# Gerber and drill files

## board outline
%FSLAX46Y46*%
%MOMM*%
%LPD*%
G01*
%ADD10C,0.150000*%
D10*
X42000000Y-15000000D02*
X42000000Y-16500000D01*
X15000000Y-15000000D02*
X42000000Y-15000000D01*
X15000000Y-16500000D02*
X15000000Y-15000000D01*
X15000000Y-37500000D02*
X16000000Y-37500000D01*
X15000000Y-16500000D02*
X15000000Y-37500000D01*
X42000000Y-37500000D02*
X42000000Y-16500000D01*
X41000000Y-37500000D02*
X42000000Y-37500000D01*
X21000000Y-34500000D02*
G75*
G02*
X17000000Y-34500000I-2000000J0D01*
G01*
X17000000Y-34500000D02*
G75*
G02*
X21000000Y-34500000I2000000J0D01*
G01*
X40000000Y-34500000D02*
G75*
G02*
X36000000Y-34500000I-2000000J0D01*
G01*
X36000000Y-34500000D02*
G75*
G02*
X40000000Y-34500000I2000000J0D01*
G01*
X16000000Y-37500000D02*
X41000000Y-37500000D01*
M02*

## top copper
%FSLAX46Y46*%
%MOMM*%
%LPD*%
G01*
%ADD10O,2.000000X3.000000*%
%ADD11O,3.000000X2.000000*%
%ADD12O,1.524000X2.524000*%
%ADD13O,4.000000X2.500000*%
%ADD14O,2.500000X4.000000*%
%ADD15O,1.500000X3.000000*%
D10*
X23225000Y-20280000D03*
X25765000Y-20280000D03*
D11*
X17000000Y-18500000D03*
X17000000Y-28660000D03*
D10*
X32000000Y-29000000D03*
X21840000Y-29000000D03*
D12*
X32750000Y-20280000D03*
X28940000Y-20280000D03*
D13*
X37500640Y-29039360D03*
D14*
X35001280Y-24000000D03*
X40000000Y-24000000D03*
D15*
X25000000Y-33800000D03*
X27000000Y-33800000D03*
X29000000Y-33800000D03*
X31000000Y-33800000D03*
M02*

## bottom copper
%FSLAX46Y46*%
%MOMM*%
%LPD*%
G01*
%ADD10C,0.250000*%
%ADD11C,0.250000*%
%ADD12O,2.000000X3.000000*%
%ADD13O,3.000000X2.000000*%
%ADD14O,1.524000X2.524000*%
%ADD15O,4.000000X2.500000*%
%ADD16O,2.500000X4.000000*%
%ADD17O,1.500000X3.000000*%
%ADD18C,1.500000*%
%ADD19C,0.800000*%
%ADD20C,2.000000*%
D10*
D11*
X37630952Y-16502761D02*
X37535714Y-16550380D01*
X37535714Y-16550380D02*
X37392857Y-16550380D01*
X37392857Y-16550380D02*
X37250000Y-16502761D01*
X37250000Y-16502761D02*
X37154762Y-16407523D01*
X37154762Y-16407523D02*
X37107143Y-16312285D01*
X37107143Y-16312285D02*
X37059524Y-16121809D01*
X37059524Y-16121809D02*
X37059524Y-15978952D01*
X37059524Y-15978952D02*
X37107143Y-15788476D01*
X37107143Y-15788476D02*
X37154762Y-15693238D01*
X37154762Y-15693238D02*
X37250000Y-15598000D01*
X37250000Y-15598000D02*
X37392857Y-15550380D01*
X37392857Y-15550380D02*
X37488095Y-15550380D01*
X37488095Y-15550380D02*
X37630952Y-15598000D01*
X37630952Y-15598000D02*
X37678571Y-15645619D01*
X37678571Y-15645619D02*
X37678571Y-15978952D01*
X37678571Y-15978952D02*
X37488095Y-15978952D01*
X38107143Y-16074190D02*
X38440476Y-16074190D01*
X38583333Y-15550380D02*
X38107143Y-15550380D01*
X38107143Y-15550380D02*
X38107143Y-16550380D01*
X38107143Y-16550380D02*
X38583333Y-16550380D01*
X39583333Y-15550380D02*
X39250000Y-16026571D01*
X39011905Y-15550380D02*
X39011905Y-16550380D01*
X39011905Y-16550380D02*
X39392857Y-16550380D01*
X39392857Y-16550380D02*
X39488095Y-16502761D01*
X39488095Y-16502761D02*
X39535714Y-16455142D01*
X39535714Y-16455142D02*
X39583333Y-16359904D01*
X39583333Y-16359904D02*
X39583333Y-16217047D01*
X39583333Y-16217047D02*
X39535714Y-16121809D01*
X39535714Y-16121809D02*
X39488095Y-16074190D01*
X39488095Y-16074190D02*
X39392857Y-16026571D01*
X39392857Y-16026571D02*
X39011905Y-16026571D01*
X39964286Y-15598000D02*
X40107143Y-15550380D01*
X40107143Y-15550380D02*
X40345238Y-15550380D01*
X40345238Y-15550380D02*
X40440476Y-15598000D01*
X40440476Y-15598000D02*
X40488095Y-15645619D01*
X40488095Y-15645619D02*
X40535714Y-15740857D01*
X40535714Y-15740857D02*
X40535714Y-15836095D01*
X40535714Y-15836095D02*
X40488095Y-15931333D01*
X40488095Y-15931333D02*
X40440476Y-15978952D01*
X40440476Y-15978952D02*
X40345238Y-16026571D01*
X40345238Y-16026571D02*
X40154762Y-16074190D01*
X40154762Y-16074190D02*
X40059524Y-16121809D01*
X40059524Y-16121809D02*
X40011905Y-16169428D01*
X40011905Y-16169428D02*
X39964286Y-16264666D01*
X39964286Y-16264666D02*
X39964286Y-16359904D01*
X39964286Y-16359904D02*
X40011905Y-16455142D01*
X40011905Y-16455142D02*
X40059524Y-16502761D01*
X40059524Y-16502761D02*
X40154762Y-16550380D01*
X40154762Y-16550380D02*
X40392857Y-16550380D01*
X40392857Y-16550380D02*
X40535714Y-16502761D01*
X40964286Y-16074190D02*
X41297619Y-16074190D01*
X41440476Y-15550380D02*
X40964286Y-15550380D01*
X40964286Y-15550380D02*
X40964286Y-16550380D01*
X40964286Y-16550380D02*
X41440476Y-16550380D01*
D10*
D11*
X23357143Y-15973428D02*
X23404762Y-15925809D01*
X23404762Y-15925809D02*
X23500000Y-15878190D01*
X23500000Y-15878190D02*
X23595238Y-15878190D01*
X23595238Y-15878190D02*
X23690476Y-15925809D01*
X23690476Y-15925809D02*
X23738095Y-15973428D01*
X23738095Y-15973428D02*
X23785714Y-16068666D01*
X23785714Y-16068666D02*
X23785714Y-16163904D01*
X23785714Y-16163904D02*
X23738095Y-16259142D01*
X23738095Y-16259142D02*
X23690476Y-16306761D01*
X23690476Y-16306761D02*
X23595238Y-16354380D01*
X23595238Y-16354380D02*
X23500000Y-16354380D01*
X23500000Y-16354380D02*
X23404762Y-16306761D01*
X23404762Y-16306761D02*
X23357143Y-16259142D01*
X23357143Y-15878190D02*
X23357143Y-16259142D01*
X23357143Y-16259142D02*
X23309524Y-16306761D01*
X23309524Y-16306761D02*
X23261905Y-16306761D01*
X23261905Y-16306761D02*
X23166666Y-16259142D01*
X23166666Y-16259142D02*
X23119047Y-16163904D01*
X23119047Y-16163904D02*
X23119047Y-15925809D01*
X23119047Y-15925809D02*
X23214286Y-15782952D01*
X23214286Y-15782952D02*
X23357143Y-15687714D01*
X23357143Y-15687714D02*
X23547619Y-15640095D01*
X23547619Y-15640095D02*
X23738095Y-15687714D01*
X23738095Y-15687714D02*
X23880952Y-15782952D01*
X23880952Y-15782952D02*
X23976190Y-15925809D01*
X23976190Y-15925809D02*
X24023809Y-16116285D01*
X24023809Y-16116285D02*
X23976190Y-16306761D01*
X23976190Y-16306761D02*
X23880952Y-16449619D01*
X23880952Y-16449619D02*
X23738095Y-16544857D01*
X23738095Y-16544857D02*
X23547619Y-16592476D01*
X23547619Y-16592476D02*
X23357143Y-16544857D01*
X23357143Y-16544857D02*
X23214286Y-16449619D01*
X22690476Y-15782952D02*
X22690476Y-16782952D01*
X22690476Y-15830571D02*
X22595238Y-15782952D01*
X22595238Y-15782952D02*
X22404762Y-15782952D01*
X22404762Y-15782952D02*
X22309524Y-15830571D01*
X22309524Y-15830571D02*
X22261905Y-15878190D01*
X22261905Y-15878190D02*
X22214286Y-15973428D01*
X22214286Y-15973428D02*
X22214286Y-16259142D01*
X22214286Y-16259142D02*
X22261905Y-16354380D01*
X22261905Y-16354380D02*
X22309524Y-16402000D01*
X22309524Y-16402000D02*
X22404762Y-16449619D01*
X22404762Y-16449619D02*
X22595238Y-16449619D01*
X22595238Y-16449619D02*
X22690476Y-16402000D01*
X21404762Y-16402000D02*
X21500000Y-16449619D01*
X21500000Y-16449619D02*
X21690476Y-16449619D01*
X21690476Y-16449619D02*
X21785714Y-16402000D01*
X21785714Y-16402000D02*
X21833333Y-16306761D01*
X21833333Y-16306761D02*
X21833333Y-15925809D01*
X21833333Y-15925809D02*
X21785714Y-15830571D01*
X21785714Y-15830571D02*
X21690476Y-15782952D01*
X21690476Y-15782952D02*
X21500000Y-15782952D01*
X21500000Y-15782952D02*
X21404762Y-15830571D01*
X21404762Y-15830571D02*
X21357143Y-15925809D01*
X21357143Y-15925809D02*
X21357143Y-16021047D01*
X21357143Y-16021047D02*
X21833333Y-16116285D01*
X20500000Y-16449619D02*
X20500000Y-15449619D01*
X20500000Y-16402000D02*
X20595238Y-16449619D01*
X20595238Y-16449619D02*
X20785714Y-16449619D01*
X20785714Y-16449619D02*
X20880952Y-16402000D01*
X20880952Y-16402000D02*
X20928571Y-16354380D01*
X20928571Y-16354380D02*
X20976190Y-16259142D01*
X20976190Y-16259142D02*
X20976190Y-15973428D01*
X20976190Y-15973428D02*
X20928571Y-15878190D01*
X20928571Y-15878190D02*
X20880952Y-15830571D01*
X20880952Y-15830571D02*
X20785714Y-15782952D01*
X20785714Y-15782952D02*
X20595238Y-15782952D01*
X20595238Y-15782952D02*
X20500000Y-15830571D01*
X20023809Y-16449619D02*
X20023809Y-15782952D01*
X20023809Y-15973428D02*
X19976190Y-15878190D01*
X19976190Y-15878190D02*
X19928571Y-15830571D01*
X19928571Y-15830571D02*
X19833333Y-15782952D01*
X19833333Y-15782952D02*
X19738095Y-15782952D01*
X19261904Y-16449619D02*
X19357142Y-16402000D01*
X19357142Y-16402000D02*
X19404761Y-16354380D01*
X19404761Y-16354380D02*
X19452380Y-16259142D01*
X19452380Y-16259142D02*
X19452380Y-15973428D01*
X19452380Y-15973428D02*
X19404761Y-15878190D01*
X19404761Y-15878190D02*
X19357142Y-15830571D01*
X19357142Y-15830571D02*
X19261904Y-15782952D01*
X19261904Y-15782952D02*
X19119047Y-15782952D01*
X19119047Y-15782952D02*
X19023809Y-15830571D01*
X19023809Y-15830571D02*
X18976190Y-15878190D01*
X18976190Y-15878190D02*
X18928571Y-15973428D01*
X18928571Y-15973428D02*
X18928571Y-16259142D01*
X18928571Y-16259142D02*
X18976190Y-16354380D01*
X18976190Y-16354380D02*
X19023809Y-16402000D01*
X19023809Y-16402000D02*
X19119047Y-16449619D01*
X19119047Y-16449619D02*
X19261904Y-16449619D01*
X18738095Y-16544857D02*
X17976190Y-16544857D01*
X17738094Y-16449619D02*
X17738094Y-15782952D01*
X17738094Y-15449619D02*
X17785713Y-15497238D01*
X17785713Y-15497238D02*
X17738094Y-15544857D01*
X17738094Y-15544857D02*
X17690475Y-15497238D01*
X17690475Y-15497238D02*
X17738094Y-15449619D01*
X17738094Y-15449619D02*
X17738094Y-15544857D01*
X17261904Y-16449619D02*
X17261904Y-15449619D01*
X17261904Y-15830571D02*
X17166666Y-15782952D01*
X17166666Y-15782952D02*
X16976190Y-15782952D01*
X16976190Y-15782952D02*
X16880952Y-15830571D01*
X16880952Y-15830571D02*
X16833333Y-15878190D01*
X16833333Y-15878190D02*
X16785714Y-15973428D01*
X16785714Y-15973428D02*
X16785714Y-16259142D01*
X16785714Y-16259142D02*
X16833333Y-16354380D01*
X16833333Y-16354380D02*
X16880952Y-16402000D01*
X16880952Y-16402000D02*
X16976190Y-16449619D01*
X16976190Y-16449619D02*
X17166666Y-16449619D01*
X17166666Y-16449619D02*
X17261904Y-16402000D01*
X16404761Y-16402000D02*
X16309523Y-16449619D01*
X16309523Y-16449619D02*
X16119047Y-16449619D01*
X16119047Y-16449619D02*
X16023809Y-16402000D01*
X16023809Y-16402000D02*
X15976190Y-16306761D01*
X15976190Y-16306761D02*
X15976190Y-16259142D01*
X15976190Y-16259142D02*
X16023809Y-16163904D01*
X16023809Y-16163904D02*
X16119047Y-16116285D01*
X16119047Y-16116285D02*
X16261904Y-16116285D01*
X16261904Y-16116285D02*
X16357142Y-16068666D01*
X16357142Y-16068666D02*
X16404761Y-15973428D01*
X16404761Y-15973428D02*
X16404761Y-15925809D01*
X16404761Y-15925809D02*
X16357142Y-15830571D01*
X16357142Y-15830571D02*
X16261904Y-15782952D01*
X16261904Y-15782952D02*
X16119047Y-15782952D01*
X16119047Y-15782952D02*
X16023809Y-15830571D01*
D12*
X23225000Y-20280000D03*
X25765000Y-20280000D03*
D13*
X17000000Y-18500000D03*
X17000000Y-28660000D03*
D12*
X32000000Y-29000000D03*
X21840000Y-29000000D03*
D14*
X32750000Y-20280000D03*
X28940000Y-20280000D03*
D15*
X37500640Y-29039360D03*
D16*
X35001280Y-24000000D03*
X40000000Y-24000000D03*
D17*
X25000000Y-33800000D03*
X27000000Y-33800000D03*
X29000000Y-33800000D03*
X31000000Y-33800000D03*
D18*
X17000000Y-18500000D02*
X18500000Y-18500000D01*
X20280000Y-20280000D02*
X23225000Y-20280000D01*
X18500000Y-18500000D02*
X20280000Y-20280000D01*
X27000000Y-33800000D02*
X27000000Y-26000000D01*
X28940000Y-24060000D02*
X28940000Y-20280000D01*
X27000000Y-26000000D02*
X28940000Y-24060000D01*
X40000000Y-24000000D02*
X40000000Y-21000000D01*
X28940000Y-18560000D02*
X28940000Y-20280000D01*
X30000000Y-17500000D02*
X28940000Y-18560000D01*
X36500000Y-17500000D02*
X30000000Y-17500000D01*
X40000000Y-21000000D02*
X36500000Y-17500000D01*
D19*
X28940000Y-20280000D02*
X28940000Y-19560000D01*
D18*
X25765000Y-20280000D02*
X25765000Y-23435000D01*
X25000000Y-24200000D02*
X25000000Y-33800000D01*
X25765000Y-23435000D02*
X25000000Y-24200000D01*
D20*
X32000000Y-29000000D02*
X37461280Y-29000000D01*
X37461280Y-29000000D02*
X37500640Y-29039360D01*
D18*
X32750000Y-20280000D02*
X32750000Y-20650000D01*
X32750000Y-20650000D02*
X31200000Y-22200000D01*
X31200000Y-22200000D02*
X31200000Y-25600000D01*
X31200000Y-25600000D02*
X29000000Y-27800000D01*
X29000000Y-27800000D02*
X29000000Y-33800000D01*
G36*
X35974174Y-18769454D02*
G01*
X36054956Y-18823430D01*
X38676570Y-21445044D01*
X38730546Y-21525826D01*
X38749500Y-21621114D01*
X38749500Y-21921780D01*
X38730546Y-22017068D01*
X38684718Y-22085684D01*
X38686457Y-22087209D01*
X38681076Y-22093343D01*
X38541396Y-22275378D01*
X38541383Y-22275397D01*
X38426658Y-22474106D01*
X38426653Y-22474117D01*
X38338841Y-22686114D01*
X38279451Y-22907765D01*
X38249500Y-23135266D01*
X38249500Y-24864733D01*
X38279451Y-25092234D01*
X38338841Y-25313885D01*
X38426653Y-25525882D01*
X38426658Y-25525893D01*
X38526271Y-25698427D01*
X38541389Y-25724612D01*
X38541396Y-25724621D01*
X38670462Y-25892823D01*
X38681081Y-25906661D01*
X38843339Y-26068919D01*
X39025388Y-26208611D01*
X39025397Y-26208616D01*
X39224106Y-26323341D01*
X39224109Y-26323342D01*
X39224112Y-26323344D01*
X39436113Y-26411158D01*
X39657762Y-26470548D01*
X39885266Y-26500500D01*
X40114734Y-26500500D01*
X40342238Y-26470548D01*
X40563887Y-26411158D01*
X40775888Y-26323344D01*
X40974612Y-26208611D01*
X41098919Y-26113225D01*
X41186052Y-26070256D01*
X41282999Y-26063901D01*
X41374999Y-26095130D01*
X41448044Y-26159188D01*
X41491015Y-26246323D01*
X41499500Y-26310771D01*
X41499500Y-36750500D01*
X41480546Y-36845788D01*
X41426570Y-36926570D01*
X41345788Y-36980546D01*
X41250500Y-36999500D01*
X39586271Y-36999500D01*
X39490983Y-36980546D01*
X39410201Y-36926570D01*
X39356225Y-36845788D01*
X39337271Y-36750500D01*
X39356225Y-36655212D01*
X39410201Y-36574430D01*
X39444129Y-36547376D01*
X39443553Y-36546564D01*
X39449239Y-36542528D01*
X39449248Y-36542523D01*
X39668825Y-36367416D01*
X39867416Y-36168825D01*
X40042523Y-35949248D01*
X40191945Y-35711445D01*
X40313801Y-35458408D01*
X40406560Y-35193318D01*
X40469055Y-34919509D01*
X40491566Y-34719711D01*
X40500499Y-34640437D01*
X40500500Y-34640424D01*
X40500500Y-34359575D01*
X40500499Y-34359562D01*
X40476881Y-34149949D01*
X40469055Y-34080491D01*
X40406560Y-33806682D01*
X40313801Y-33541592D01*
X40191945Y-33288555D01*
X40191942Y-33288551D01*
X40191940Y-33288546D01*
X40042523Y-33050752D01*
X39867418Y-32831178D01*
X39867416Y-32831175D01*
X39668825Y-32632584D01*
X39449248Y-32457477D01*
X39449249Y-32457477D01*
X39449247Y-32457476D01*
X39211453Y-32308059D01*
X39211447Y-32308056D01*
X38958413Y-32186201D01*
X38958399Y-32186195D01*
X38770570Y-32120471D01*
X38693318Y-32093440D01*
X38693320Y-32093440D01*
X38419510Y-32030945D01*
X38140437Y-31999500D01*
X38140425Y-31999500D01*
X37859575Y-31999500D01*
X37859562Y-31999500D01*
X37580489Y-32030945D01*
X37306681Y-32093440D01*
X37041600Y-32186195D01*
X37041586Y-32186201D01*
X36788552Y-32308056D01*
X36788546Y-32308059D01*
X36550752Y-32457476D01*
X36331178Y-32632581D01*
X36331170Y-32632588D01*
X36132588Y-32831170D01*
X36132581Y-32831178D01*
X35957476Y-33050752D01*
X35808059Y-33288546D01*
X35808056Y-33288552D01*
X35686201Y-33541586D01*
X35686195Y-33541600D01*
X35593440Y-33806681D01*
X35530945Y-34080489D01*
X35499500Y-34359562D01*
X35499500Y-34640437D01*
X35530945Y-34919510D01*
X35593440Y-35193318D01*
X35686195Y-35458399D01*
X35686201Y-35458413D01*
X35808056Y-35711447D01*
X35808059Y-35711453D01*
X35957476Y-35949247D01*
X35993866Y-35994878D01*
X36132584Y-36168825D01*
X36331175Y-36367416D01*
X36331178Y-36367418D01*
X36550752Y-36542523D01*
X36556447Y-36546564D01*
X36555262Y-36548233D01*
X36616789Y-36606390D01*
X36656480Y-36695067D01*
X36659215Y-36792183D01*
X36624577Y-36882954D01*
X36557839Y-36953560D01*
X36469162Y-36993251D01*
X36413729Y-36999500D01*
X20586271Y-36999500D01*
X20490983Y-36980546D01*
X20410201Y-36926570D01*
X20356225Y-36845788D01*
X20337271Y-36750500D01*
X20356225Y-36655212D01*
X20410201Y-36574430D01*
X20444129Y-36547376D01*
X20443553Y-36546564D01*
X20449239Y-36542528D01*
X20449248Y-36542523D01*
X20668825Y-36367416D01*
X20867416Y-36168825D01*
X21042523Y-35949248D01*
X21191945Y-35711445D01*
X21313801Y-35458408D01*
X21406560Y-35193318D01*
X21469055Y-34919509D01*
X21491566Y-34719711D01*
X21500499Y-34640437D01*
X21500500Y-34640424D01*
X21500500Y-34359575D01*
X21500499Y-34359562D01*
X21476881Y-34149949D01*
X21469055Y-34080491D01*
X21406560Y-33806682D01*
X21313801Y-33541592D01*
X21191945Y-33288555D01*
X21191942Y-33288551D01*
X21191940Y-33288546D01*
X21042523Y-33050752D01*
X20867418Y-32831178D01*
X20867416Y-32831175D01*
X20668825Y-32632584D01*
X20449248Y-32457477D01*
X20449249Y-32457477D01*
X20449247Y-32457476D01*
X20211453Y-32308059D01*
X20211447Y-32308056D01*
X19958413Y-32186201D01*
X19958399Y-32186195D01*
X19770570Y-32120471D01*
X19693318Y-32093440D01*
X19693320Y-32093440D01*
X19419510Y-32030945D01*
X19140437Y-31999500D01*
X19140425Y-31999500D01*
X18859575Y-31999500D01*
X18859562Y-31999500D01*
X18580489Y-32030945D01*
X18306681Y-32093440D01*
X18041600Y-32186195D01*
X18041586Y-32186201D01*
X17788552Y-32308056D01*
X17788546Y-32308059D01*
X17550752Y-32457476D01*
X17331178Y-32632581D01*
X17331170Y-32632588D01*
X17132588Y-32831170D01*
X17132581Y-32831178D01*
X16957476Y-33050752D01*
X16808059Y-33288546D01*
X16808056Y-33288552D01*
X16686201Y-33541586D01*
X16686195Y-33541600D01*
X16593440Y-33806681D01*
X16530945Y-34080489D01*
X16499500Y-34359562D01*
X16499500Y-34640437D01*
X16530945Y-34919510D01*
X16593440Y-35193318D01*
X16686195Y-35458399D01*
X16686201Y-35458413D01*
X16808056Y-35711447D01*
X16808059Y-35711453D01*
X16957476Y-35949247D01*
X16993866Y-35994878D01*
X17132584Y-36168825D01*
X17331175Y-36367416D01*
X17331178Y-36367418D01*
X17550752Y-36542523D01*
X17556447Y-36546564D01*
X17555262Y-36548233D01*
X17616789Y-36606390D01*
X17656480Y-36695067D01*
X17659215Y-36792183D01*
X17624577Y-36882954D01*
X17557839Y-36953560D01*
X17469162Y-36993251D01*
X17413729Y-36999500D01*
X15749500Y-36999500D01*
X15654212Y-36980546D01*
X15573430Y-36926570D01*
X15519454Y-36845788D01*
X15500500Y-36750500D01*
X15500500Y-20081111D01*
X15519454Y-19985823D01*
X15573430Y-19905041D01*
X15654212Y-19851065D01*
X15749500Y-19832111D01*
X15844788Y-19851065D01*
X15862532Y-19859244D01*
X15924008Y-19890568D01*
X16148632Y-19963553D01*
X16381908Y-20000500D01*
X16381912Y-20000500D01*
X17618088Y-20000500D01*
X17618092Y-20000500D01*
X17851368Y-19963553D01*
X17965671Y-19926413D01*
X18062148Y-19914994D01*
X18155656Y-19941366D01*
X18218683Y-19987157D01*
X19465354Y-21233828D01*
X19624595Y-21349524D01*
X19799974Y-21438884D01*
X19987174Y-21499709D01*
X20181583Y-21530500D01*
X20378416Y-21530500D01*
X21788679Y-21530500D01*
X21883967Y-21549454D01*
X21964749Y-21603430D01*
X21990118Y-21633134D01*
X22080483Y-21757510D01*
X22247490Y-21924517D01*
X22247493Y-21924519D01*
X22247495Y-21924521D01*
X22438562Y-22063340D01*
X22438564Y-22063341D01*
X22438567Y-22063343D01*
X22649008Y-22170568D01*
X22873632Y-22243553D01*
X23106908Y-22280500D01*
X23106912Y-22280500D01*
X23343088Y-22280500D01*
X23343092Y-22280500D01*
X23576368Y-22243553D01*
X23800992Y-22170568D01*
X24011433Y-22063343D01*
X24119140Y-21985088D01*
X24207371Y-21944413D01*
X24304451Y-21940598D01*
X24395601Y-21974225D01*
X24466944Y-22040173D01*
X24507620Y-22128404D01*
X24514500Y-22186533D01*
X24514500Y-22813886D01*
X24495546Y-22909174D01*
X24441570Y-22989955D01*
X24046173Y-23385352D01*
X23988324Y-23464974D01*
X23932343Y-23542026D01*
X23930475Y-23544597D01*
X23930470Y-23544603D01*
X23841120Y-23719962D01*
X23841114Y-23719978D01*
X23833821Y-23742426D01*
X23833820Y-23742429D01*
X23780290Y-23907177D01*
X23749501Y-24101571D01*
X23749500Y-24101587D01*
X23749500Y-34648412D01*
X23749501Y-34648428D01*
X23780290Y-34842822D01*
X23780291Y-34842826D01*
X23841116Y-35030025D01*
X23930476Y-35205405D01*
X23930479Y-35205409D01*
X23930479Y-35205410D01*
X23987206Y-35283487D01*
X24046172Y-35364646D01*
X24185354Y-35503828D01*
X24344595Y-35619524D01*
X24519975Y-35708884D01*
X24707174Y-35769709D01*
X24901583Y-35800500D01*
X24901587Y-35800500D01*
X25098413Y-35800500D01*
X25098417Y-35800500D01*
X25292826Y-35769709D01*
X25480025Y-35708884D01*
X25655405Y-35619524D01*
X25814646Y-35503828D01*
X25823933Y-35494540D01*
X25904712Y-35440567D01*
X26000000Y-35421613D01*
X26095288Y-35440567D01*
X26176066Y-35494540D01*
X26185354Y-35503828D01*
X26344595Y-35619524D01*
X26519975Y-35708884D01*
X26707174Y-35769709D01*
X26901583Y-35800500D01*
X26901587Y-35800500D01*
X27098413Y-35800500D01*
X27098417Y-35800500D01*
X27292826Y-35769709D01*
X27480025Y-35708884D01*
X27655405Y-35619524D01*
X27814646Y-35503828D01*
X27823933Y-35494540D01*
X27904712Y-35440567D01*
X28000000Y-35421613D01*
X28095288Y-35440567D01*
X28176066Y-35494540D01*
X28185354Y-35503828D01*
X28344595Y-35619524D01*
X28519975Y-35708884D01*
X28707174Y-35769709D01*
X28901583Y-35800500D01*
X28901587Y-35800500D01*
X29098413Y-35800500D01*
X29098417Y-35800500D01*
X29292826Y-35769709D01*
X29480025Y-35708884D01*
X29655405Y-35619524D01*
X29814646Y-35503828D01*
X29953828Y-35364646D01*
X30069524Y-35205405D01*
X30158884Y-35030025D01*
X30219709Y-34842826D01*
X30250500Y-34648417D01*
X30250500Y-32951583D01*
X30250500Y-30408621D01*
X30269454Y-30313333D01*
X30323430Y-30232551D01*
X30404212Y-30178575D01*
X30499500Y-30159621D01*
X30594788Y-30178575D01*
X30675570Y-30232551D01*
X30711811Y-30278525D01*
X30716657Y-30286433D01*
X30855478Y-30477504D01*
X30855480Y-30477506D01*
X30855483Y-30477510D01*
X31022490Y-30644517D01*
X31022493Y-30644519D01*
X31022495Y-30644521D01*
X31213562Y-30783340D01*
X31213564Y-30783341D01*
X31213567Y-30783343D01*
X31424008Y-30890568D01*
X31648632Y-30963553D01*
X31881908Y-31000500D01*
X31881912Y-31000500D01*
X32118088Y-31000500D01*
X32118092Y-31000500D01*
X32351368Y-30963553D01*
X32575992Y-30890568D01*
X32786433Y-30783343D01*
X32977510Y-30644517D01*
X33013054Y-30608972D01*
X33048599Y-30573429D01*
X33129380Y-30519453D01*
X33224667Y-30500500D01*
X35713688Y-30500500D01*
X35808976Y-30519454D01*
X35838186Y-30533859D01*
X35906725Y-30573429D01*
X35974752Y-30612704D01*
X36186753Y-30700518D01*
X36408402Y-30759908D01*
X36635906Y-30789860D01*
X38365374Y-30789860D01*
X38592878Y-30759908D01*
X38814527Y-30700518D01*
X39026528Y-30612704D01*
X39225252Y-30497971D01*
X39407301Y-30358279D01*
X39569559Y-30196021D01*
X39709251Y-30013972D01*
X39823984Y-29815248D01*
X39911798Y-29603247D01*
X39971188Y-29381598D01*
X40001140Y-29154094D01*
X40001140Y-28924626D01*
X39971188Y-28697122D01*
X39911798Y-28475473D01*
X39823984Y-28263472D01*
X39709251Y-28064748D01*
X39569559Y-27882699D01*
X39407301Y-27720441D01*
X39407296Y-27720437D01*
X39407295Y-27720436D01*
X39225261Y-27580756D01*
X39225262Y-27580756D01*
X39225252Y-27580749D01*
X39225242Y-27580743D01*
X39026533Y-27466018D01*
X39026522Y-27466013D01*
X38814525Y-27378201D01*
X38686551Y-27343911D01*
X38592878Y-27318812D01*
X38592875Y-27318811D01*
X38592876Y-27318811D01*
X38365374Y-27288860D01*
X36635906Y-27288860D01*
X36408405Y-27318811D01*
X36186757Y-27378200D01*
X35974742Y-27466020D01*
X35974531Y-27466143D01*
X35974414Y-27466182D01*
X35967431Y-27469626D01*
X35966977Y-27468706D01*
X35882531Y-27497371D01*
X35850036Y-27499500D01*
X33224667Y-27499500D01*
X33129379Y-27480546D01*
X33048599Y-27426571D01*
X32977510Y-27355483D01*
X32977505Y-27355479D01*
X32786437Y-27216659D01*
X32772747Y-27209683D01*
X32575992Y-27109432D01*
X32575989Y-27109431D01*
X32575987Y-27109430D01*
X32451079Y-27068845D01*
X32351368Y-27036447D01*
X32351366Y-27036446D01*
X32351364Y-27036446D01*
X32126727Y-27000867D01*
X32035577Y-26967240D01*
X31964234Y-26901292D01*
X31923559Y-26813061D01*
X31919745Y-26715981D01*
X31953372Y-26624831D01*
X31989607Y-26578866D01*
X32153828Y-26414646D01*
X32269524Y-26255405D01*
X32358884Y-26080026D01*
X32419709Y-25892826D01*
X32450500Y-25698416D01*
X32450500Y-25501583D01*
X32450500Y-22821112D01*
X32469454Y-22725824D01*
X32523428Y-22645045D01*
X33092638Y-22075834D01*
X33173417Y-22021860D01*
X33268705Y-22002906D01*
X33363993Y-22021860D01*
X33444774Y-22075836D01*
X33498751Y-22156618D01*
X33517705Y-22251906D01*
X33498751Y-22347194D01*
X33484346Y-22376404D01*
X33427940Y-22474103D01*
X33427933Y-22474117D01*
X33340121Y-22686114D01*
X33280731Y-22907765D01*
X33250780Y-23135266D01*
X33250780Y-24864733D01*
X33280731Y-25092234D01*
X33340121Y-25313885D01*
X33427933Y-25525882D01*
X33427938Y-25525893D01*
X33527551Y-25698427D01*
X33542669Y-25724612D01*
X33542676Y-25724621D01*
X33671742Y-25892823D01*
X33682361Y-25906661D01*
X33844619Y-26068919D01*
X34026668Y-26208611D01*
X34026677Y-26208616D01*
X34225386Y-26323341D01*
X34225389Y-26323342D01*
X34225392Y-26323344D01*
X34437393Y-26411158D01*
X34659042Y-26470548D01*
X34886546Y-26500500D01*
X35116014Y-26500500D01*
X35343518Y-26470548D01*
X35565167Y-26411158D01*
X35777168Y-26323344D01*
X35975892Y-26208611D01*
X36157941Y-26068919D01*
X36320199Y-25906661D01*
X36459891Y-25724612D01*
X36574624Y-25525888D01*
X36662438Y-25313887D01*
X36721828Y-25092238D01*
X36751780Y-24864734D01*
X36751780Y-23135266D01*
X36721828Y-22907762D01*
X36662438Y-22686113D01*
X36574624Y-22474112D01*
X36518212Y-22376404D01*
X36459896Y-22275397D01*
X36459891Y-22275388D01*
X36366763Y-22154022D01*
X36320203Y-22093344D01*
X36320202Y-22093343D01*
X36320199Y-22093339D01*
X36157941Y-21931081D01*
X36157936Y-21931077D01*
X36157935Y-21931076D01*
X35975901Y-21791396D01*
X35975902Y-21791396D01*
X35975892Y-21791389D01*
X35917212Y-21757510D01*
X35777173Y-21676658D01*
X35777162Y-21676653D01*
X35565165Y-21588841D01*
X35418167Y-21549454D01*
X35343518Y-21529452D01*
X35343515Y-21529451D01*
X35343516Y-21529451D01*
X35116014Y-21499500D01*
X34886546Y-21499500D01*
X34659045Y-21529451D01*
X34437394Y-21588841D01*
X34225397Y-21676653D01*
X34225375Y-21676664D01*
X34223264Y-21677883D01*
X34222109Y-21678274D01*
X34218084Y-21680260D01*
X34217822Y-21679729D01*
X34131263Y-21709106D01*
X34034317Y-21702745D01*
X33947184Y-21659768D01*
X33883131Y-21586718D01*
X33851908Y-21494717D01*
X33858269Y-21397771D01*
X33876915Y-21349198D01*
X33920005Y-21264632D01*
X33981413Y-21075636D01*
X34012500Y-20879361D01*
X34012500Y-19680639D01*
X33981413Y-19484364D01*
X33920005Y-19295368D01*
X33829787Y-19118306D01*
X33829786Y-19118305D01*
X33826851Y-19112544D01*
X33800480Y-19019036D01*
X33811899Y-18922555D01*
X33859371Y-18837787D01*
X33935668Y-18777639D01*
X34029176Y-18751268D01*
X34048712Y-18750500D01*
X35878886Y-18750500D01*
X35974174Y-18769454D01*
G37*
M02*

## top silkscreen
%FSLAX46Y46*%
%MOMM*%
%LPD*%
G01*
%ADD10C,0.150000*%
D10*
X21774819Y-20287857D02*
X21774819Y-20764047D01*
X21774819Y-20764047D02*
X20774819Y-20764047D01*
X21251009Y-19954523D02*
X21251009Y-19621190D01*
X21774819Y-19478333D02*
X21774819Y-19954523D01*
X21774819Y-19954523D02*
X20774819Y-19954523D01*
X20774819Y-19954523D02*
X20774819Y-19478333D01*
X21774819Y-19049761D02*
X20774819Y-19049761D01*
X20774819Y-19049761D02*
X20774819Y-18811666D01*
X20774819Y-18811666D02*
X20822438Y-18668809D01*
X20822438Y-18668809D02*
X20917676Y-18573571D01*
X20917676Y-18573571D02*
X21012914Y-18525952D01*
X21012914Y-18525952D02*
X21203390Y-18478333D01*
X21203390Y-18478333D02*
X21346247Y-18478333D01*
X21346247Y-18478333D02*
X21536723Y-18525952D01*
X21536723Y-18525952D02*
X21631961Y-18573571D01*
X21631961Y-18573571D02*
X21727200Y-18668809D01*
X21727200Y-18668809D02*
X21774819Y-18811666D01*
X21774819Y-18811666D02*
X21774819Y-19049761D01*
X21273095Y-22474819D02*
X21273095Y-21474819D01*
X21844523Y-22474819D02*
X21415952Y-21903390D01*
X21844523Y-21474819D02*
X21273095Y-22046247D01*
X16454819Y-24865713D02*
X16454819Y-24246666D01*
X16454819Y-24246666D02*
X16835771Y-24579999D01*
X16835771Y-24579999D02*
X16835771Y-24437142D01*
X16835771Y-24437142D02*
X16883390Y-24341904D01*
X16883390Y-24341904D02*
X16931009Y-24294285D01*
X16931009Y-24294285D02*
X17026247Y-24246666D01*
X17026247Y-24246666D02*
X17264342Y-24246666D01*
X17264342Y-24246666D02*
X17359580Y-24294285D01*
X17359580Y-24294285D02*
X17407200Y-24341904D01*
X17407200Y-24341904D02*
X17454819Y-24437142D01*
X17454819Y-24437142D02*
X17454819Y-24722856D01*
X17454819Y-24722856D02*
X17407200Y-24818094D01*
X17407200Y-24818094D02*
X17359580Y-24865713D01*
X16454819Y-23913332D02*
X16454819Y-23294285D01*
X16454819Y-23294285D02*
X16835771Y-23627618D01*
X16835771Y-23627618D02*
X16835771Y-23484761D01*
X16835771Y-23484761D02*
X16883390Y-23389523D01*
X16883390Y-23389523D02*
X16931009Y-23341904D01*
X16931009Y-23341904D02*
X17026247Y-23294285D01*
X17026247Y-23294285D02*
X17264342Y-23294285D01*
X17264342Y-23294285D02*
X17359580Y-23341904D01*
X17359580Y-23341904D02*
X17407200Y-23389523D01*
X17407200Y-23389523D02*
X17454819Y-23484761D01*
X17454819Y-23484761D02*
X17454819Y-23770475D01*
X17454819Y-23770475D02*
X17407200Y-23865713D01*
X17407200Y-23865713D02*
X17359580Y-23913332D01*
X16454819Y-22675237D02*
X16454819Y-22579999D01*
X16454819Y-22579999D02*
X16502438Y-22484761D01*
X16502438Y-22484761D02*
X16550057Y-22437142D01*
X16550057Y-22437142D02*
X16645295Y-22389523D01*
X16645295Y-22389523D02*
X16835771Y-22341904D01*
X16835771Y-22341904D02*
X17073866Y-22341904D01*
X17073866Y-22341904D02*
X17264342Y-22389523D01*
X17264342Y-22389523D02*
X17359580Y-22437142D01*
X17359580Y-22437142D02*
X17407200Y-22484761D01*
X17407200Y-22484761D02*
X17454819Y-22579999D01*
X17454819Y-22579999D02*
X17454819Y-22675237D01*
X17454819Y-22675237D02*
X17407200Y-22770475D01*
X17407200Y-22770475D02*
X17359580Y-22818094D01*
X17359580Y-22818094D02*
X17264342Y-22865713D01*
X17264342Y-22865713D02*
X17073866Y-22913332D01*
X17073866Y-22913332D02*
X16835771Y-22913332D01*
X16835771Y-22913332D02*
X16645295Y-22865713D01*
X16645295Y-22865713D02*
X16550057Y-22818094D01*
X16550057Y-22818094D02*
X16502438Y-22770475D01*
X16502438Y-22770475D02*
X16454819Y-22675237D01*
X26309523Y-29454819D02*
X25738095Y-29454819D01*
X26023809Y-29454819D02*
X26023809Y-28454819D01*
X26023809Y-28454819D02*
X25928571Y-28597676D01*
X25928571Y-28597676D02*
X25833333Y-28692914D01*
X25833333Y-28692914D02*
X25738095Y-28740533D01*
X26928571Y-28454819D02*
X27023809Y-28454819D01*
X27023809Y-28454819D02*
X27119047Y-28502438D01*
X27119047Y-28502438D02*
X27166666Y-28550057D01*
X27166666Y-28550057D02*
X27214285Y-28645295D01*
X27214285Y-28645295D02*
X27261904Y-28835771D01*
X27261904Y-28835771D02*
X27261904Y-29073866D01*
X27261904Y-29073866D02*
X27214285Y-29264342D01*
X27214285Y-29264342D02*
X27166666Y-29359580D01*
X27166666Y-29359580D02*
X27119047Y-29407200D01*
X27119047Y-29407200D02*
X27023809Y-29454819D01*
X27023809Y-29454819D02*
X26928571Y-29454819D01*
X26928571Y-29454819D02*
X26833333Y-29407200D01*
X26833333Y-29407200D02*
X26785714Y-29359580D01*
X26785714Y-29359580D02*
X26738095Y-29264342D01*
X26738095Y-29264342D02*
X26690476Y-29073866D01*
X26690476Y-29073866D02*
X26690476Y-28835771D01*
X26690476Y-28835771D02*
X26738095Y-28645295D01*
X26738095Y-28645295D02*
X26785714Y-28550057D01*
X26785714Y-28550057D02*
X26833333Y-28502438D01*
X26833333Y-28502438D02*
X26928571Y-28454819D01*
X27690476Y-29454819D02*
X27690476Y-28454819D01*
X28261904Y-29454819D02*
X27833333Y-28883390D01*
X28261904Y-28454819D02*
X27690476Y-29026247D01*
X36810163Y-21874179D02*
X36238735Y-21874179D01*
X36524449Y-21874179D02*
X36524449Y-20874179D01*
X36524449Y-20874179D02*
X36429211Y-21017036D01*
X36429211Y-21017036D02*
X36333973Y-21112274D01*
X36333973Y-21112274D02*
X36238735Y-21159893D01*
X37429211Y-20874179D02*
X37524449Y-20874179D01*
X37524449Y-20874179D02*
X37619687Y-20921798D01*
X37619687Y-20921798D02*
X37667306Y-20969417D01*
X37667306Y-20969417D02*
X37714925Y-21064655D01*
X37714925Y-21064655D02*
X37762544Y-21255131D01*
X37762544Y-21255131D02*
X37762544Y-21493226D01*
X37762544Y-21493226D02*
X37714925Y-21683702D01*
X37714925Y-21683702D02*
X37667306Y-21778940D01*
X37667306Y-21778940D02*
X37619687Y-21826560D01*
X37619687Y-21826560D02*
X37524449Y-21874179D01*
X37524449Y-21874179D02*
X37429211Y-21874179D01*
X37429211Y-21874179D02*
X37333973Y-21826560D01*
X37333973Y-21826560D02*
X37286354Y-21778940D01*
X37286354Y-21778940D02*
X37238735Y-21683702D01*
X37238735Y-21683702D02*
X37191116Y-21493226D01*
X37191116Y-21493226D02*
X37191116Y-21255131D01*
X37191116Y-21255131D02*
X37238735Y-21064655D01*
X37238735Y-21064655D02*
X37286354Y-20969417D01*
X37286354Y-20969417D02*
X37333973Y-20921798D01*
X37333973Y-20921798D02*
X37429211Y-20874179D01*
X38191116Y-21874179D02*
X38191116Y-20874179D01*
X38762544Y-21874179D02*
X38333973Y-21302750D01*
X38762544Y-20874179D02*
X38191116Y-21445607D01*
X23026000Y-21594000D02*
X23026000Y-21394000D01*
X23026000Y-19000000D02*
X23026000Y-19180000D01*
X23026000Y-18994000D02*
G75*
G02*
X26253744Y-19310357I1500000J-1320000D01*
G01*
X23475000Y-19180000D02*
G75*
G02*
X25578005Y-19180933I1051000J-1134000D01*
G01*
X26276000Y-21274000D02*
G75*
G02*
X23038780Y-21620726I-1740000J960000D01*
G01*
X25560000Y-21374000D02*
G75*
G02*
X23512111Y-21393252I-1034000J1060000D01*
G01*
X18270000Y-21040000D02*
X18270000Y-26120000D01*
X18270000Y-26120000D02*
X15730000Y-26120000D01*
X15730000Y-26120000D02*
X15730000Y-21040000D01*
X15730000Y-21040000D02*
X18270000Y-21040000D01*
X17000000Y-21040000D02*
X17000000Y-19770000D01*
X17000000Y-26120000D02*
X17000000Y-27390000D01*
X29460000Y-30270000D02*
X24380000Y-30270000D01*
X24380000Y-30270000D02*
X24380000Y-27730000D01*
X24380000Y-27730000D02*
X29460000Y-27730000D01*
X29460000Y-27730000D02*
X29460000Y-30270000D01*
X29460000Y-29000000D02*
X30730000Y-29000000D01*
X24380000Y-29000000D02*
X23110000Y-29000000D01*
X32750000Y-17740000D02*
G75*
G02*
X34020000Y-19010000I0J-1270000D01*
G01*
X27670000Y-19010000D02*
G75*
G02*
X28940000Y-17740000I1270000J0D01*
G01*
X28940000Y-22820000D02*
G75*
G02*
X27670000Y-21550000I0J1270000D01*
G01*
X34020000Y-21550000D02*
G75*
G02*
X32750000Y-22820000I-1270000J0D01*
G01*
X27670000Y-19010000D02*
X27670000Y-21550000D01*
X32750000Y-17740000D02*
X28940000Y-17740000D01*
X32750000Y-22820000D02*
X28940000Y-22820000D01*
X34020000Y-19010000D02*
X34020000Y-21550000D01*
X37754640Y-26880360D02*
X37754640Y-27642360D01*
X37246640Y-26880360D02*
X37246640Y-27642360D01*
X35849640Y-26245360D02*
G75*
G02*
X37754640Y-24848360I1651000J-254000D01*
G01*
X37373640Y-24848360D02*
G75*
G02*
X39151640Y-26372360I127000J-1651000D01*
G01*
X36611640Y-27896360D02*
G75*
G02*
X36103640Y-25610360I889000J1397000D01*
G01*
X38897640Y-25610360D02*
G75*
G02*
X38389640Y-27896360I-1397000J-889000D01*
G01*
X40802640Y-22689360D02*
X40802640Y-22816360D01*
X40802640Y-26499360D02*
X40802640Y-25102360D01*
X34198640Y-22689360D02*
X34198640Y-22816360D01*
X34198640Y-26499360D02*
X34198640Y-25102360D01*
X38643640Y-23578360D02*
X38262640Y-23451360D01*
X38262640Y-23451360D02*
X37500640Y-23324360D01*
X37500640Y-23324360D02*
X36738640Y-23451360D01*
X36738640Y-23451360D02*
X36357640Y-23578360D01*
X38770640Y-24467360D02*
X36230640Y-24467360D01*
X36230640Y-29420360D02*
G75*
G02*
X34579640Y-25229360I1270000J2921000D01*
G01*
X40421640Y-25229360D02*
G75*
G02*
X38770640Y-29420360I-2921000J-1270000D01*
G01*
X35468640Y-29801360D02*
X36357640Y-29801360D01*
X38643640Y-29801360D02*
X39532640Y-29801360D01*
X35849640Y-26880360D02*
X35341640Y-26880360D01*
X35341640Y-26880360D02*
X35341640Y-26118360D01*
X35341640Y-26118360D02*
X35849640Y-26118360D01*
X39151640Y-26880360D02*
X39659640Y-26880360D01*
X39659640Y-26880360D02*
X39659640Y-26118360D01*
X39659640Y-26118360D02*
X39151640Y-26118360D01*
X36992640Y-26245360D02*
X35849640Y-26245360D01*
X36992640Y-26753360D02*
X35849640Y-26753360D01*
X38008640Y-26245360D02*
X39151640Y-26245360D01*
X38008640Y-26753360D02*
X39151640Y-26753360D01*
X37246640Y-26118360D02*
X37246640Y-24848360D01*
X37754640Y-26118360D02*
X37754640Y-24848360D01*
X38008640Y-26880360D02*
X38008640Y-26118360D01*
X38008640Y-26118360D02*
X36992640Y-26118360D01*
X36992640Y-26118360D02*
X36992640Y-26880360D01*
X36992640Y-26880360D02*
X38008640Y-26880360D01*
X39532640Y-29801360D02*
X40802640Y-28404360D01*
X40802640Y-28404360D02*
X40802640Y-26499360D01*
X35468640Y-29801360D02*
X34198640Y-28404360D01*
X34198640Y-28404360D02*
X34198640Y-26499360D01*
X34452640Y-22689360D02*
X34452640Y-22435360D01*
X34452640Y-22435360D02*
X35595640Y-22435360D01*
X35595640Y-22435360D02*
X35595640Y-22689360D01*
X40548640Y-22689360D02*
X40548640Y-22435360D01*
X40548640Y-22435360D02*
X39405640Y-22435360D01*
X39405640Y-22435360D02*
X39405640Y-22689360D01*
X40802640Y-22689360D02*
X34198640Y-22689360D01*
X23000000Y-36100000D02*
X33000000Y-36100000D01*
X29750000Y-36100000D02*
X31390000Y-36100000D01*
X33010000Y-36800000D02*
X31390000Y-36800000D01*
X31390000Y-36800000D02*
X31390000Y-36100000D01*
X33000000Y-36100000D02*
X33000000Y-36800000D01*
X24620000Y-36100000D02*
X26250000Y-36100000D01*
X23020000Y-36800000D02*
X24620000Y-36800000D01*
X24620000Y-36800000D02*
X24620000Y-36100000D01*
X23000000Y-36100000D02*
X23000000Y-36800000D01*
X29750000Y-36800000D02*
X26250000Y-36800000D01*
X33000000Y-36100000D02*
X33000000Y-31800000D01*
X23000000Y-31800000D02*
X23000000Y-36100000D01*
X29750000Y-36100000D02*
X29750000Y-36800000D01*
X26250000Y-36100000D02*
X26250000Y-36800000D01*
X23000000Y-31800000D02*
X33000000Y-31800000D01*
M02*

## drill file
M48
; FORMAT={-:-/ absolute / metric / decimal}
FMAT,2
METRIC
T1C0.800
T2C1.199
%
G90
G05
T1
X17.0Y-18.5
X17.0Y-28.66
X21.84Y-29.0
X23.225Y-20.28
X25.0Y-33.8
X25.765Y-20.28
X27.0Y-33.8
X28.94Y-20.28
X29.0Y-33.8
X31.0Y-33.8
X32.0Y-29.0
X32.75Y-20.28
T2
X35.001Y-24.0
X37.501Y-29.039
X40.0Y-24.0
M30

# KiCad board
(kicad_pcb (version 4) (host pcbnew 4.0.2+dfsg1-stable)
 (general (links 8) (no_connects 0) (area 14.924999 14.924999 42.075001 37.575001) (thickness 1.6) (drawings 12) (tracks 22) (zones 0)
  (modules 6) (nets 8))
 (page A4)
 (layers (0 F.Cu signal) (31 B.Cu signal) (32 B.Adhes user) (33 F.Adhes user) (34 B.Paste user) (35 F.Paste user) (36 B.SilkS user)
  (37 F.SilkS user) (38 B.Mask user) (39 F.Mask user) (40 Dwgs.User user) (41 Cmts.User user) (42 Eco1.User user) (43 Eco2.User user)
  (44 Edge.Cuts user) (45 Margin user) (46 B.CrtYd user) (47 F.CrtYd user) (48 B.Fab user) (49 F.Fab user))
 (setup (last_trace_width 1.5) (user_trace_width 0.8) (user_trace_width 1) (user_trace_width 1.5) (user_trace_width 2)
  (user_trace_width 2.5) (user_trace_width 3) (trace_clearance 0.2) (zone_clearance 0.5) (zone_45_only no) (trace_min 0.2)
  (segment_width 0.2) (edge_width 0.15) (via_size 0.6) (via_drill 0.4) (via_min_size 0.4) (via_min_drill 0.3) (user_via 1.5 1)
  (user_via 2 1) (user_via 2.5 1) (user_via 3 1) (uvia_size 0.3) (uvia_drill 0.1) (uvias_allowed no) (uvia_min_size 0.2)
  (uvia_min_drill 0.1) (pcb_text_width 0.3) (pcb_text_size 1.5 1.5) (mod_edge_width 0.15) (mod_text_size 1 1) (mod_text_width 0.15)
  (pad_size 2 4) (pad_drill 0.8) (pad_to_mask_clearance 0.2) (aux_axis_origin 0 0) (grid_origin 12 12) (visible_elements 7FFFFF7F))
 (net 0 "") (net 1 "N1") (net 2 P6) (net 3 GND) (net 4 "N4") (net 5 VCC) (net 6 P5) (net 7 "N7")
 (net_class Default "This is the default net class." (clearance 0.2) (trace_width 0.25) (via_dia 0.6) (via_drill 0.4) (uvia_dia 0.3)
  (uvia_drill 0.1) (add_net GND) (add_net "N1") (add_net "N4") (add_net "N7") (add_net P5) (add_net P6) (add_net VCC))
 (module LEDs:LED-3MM (layer F.Cu) (at 23.225 20.28)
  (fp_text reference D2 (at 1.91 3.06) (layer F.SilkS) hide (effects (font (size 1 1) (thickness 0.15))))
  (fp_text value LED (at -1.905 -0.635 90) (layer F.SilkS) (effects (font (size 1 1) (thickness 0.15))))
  (fp_line (start -0.199 1.314) (end -0.199 1.114) (layer F.SilkS) (width 0.15))
  (fp_line (start -0.199 -1.28) (end -0.199 -1.1) (layer F.SilkS) (width 0.15))
  (fp_arc (start 1.301 0.034) (end -0.199 -1.286) (angle 108.5) (layer F.SilkS) (width 0.15))
  (fp_arc (start 1.301 0.034) (end 0.25 -1.1) (angle 85.7) (layer F.SilkS) (width 0.15))
  (fp_arc (start 1.311 0.034) (end 3.051 0.994) (angle 110) (layer F.SilkS) (width 0.15))
  (fp_arc (start 1.301 0.034) (end 2.335 1.094) (angle 87.5) (layer F.SilkS) (width 0.15))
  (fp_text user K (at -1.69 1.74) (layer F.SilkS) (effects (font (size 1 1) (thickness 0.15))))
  (pad 1 thru_hole oval (at 0 0 90) (size 3 2) (drill 0.8) (layers *.Cu) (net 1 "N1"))
  (pad 2 thru_hole oval (at 2.54 0) (size 2 3) (drill 0.8) (layers *.Cu) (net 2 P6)))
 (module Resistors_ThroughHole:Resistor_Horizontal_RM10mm (layer F.Cu) (at 17 18.5 270)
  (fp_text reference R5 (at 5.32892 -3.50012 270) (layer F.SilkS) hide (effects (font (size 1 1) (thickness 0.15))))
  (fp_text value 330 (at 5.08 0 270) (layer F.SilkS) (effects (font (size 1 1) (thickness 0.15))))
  (fp_line (start 2.54 -1.27) (end 7.62 -1.27) (layer F.SilkS) (width 0.15))
  (fp_line (start 7.62 -1.27) (end 7.62 1.27) (layer F.SilkS) (width 0.15))
  (fp_line (start 7.62 1.27) (end 2.54 1.27) (layer F.SilkS) (width 0.15))
  (fp_line (start 2.54 1.27) (end 2.54 -1.27) (layer F.SilkS) (width 0.15))
  (fp_line (start 2.54 0) (end 1.27 0) (layer F.SilkS) (width 0.15))
  (fp_line (start 7.62 0) (end 8.89 0) (layer F.SilkS) (width 0.15))
  (pad 1 thru_hole oval (at 0 0 270) (size 2 3) (drill 0.8) (layers *.Cu) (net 1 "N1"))
  (pad 2 thru_hole oval (at 10.16 0 270) (size 2 3) (drill 0.8) (layers *.Cu) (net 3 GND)))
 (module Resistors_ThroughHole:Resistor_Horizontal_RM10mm (layer F.Cu) (at 32 29 180)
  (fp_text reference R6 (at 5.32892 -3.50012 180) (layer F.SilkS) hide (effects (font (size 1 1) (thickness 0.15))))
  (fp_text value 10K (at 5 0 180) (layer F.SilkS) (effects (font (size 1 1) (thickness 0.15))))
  (fp_line (start 2.54 -1.27) (end 7.62 -1.27) (layer F.SilkS) (width 0.15))
  (fp_line (start 7.62 -1.27) (end 7.62 1.27) (layer F.SilkS) (width 0.15))
  (fp_line (start 7.62 1.27) (end 2.54 1.27) (layer F.SilkS) (width 0.15))
  (fp_line (start 2.54 1.27) (end 2.54 -1.27) (layer F.SilkS) (width 0.15))
  (fp_line (start 2.54 0) (end 1.27 0) (layer F.SilkS) (width 0.15))
  (fp_line (start 7.62 0) (end 8.89 0) (layer F.SilkS) (width 0.15))
  (pad 1 thru_hole oval (at 0 0 180) (size 2 3) (drill 0.8) (layers *.Cu) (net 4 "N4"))
  (pad 2 thru_hole oval (at 10.16 0 180) (size 2 3) (drill 0.8) (layers *.Cu) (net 3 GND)))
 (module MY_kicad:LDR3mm (layer F.Cu) (at 32.75 20.28 180)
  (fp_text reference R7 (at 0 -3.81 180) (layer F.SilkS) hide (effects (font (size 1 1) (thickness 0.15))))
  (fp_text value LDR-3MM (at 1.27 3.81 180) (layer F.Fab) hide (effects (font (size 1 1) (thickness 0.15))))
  (fp_arc (start 0 1.27) (end 0 2.54) (angle 90) (layer F.SilkS) (width 0.15))
  (fp_arc (start 3.81 1.27) (end 5.08 1.27) (angle 90) (layer F.SilkS) (width 0.15))
  (fp_arc (start 3.81 -1.27) (end 3.81 -2.54) (angle 90) (layer F.SilkS) (width 0.15))
  (fp_arc (start 0 -1.27) (end -1.27 -1.27) (angle 90) (layer F.SilkS) (width 0.15))
  (fp_line (start 5.08 1.27) (end 5.08 -1.27) (layer F.SilkS) (width 0.15))
  (fp_line (start 0 2.54) (end 3.81 2.54) (layer F.SilkS) (width 0.15))
  (fp_line (start 0 -2.54) (end 3.81 -2.54) (layer F.SilkS) (width 0.15))
  (fp_line (start -1.27 1.27) (end -1.27 -1.27) (layer F.SilkS) (width 0.15))
  (pad 1 thru_hole oval (at 0 0 180) (size 1.524 2.524) (drill 0.8) (layers *.Cu) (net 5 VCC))
  (pad 2 thru_hole oval (at 3.81 0 180) (size 1.524 2.524) (drill 0.8) (layers *.Cu) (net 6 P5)))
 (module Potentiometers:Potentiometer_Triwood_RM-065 (layer F.Cu) (at 40 24 180)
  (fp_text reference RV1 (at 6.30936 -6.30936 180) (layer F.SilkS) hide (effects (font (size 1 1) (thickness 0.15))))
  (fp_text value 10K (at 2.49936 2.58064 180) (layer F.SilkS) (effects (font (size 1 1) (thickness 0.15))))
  (fp_line (start 2.24536 -2.88036) (end 2.24536 -3.64236) (layer F.SilkS) (width 0.15))
  (fp_line (start 2.75336 -2.88036) (end 2.75336 -3.64236) (layer F.SilkS) (width 0.15))
  (fp_arc (start 2.49936 -2.49936) (end 4.15036 -2.24536) (angle 90) (layer F.SilkS) (width 0.15))
  (fp_arc (start 2.49936 -2.49936) (end 2.62636 -0.84836) (angle 90) (layer F.SilkS) (width 0.15))
  (fp_arc (start 2.49936 -2.49936) (end 3.38836 -3.89636) (angle 90) (layer F.SilkS) (width 0.15))
  (fp_arc (start 2.49936 -2.49936) (end 1.10236 -1.61036) (angle 90) (layer F.SilkS) (width 0.15))
  (fp_line (start -0.80264 1.31064) (end -0.80264 1.18364) (layer F.SilkS) (width 0.15))
  (fp_line (start -0.80264 -2.49936) (end -0.80264 -1.10236) (layer F.SilkS) (width 0.15))
  (fp_line (start 5.80136 1.31064) (end 5.80136 1.18364) (layer F.SilkS) (width 0.15))
  (fp_line (start 5.80136 -2.49936) (end 5.80136 -1.10236) (layer F.SilkS) (width 0.15))
  (fp_line (start 1.35636 0.42164) (end 1.73736 0.54864) (layer F.SilkS) (width 0.15))
  (fp_line (start 1.73736 0.54864) (end 2.49936 0.67564) (layer F.SilkS) (width 0.15))
  (fp_line (start 2.49936 0.67564) (end 3.26136 0.54864) (layer F.SilkS) (width 0.15))
  (fp_line (start 3.26136 0.54864) (end 3.64236 0.42164) (layer F.SilkS) (width 0.15))
  (fp_line (start 1.22936 -0.46736) (end 3.76936 -0.46736) (layer F.SilkS) (width 0.15))
  (fp_arc (start 2.49936 -2.49936) (end 3.76936 -5.42036) (angle 90) (layer F.SilkS) (width 0.15))
  (fp_arc (start 2.49936 -2.49936) (end -0.42164 -1.22936) (angle 90) (layer F.SilkS) (width 0.15))
  (fp_line (start 4.53136 -5.80136) (end 3.64236 -5.80136) (layer F.SilkS) (width 0.15))
  (fp_line (start 1.35636 -5.80136) (end 0.46736 -5.80136) (layer F.SilkS) (width 0.15))
  (fp_line (start 4.15036 -2.88036) (end 4.65836 -2.88036) (layer F.SilkS) (width 0.15))
  (fp_line (start 4.65836 -2.88036) (end 4.65836 -2.11836) (layer F.SilkS) (width 0.15))
  (fp_line (start 4.65836 -2.11836) (end 4.15036 -2.11836) (layer F.SilkS) (width 0.15))
  (fp_line (start 0.84836 -2.88036) (end 0.34036 -2.88036) (layer F.SilkS) (width 0.15))
  (fp_line (start 0.34036 -2.88036) (end 0.34036 -2.11836) (layer F.SilkS) (width 0.15))
  (fp_line (start 0.34036 -2.11836) (end 0.84836 -2.11836) (layer F.SilkS) (width 0.15))
  (fp_line (start 3.00736 -2.24536) (end 4.15036 -2.24536) (layer F.SilkS) (width 0.15))
  (fp_line (start 3.00736 -2.75336) (end 4.15036 -2.75336) (layer F.SilkS) (width 0.15))
  (fp_line (start 1.99136 -2.24536) (end 0.84836 -2.24536) (layer F.SilkS) (width 0.15))
  (fp_line (start 1.99136 -2.75336) (end 0.84836 -2.75336) (layer F.SilkS) (width 0.15))
  (fp_line (start 2.75336 -2.11836) (end 2.75336 -0.84836) (layer F.SilkS) (width 0.15))
  (fp_line (start 2.24536 -2.11836) (end 2.24536 -0.84836) (layer F.SilkS) (width 0.15))
  (fp_line (start 1.99136 -2.88036) (end 1.99136 -2.11836) (layer F.SilkS) (width 0.15))
  (fp_line (start 1.99136 -2.11836) (end 3.00736 -2.11836) (layer F.SilkS) (width 0.15))
  (fp_line (start 3.00736 -2.11836) (end 3.00736 -2.88036) (layer F.SilkS) (width 0.15))
  (fp_line (start 3.00736 -2.88036) (end 1.99136 -2.88036) (layer F.SilkS) (width 0.15))
  (fp_line (start 0.46736 -5.80136) (end -0.80264 -4.40436) (layer F.SilkS) (width 0.15))
  (fp_line (start -0.80264 -4.40436) (end -0.80264 -2.49936) (layer F.SilkS) (width 0.15))
  (fp_line (start 4.53136 -5.80136) (end 5.80136 -4.40436) (layer F.SilkS) (width 0.15))
  (fp_line (start 5.80136 -4.40436) (end 5.80136 -2.49936) (layer F.SilkS) (width 0.15))
  (fp_line (start 5.54736 1.31064) (end 5.54736 1.56464) (layer F.SilkS) (width 0.15))
  (fp_line (start 5.54736 1.56464) (end 4.40436 1.56464) (layer F.SilkS) (width 0.15))
  (fp_line (start 4.40436 1.56464) (end 4.40436 1.31064) (layer F.SilkS) (width 0.15))
  (fp_line (start -0.54864 1.31064) (end -0.54864 1.56464) (layer F.SilkS) (width 0.15))
  (fp_line (start -0.54864 1.56464) (end 0.59436 1.56464) (layer F.SilkS) (width 0.15))
  (fp_line (start 0.59436 1.56464) (end 0.59436 1.31064) (layer F.SilkS) (width 0.15))
  (fp_line (start -0.80264 1.31064) (end 5.80136 1.31064) (layer F.SilkS) (width 0.15))
  (pad 2 thru_hole oval (at 2.49936 -5.03936 180) (size 4 2.5) (drill 1.19888) (layers *.Cu) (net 4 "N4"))
  (pad 3 thru_hole oval (at 4.99872 0 180) (size 2.5 4) (drill 1.19888) (layers *.Cu) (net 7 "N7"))
  (pad 1 thru_hole oval (at 0 0 180) (size 2.5 4) (drill 1.19888) (layers *.Cu) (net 6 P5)))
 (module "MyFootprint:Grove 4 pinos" (layer F.Cu) (at 28 33.8)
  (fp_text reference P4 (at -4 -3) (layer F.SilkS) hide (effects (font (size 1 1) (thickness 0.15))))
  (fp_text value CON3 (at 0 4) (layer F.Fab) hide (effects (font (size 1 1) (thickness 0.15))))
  (fp_line (start -5 2.3) (end 5 2.3) (layer F.SilkS) (width 0.15))
  (fp_line (start 1.75 2.3) (end 3.39 2.3) (layer F.SilkS) (width 0.15))
  (fp_line (start 5.01 3) (end 3.39 3) (layer F.SilkS) (width 0.15))
  (fp_line (start 3.39 3) (end 3.39 2.3) (layer F.SilkS) (width 0.15))
  (fp_line (start 5 2.3) (end 5 3) (layer F.SilkS) (width 0.15))
  (fp_line (start -3.38 2.3) (end -1.75 2.3) (layer F.SilkS) (width 0.15))
  (fp_line (start -4.98 3) (end -3.38 3) (layer F.SilkS) (width 0.15))
  (fp_line (start -3.38 3) (end -3.38 2.3) (layer F.SilkS) (width 0.15))
  (fp_line (start -5 2.3) (end -5 3) (layer F.SilkS) (width 0.15))
  (fp_line (start 1.75 3) (end -1.75 3) (layer F.SilkS) (width 0.15))
  (fp_line (start 5 2.3) (end 5 -2) (layer F.SilkS) (width 0.15))
  (fp_line (start -5 -2) (end -5 2.3) (layer F.SilkS) (width 0.15))
  (fp_line (start 1.75 2.3) (end 1.75 3) (layer F.SilkS) (width 0.15))
  (fp_line (start -1.75 2.3) (end -1.75 3) (layer F.SilkS) (width 0.15))
  (fp_line (start -5 -2) (end 5 -2) (layer F.SilkS) (width 0.15))
  (pad 1 thru_hole oval (at -3 0) (size 1.5 3) (drill 0.8) (layers *.Cu) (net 2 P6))
  (pad 2 thru_hole oval (at -1 0) (size 1.5 3) (drill 0.8) (layers *.Cu) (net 6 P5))
  (pad 3 thru_hole oval (at 1 0) (size 1.5 3) (drill 0.8) (layers *.Cu) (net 5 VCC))
  (pad 4 thru_hole oval (at 3 0) (size 1.5 3) (drill 0.8) (layers *.Cu) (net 3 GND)))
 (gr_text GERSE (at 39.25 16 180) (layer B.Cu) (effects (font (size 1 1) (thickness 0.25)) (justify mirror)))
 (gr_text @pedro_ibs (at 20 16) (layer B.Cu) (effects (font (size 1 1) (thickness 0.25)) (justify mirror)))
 (gr_line (start 42 15) (end 42 16.5) (angle 90) (layer Edge.Cuts) (width 0.15))
 (gr_line (start 15 15) (end 42 15) (angle 90) (layer Edge.Cuts) (width 0.15))
 (gr_line (start 15 16.5) (end 15 15) (angle 90) (layer Edge.Cuts) (width 0.15))
 (gr_line (start 15 37.5) (end 16 37.5) (angle 90) (layer Edge.Cuts) (width 0.15))
 (gr_line (start 15 16.5) (end 15 37.5) (angle 90) (layer Edge.Cuts) (width 0.15))
 (gr_line (start 42 37.5) (end 42 16.5) (angle 90) (layer Edge.Cuts) (width 0.15))
 (gr_line (start 41 37.5) (end 42 37.5) (angle 90) (layer Edge.Cuts) (width 0.15))
 (gr_circle (center 19 34.5) (end 21 34.5) (layer Edge.Cuts) (width 0.15))
 (gr_circle (center 38 34.5) (end 40 34.5) (layer Edge.Cuts) (width 0.15))
 (gr_line (start 16 37.5) (end 41 37.5) (angle 90) (layer Edge.Cuts) (width 0.15))
 (segment (start 17 18.5) (end 18.5 18.5) (width 1.5) (layer B.Cu) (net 1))
 (segment (start 20.28 20.28) (end 23.225 20.28) (width 1.5) (layer B.Cu) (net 1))
 (segment (start 18.5 18.5) (end 20.28 20.28) (width 1.5) (layer B.Cu) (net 1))
 (segment (start 27 33.8) (end 27 26) (width 1.5) (layer B.Cu) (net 6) (status 400000))
 (segment (start 28.94 24.06) (end 28.94 20.28) (width 1.5) (layer B.Cu) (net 6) (status 800000))
 (segment (start 27 26) (end 28.94 24.06) (width 1.5) (layer B.Cu) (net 6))
 (segment (start 40 24) (end 40 21) (width 1.5) (layer B.Cu) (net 6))
 (segment (start 28.94 18.56) (end 28.94 20.28) (width 1.5) (layer B.Cu) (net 6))
 (segment (start 30 17.5) (end 28.94 18.56) (width 1.5) (layer B.Cu) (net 6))
 (segment (start 36.5 17.5) (end 30 17.5) (width 1.5) (layer B.Cu) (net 6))
 (segment (start 40 21) (end 36.5 17.5) (width 1.5) (layer B.Cu) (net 6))
 (segment (start 28.94 20.28) (end 28.94 19.56) (width 0.8) (layer B.Cu) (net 6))
 (segment (start 25.765 20.28) (end 25.765 23.435) (width 1.5) (layer B.Cu) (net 2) (status 400000))
 (segment (start 25 24.2) (end 25 33.8) (width 1.5) (layer B.Cu) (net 2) (status 800000))
 (segment (start 25.765 23.435) (end 25 24.2) (width 1.5) (layer B.Cu) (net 2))
 (segment (start 32 29) (end 37.46128 29) (width 2) (layer B.Cu) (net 4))
 (segment (start 37.46128 29) (end 37.50064 29.03936) (width 2) (layer B.Cu) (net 4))
 (segment (start 32.75 20.28) (end 32.75 20.65) (width 1.5) (layer B.Cu) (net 5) (status C00000))
 (segment (start 32.75 20.65) (end 31.2 22.2) (width 1.5) (layer B.Cu) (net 5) (status 400000))
 (segment (start 31.2 22.2) (end 31.2 25.6) (width 1.5) (layer B.Cu) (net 5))
 (segment (start 31.2 25.6) (end 29 27.8) (width 1.5) (layer B.Cu) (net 5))
 (segment (start 29 27.8) (end 29 33.8) (width 1.5) (layer B.Cu) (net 5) (status 800000))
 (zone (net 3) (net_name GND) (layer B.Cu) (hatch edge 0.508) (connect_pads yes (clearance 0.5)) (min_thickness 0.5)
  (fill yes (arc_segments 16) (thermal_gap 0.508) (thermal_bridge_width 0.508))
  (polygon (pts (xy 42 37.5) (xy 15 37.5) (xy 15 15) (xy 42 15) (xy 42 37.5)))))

